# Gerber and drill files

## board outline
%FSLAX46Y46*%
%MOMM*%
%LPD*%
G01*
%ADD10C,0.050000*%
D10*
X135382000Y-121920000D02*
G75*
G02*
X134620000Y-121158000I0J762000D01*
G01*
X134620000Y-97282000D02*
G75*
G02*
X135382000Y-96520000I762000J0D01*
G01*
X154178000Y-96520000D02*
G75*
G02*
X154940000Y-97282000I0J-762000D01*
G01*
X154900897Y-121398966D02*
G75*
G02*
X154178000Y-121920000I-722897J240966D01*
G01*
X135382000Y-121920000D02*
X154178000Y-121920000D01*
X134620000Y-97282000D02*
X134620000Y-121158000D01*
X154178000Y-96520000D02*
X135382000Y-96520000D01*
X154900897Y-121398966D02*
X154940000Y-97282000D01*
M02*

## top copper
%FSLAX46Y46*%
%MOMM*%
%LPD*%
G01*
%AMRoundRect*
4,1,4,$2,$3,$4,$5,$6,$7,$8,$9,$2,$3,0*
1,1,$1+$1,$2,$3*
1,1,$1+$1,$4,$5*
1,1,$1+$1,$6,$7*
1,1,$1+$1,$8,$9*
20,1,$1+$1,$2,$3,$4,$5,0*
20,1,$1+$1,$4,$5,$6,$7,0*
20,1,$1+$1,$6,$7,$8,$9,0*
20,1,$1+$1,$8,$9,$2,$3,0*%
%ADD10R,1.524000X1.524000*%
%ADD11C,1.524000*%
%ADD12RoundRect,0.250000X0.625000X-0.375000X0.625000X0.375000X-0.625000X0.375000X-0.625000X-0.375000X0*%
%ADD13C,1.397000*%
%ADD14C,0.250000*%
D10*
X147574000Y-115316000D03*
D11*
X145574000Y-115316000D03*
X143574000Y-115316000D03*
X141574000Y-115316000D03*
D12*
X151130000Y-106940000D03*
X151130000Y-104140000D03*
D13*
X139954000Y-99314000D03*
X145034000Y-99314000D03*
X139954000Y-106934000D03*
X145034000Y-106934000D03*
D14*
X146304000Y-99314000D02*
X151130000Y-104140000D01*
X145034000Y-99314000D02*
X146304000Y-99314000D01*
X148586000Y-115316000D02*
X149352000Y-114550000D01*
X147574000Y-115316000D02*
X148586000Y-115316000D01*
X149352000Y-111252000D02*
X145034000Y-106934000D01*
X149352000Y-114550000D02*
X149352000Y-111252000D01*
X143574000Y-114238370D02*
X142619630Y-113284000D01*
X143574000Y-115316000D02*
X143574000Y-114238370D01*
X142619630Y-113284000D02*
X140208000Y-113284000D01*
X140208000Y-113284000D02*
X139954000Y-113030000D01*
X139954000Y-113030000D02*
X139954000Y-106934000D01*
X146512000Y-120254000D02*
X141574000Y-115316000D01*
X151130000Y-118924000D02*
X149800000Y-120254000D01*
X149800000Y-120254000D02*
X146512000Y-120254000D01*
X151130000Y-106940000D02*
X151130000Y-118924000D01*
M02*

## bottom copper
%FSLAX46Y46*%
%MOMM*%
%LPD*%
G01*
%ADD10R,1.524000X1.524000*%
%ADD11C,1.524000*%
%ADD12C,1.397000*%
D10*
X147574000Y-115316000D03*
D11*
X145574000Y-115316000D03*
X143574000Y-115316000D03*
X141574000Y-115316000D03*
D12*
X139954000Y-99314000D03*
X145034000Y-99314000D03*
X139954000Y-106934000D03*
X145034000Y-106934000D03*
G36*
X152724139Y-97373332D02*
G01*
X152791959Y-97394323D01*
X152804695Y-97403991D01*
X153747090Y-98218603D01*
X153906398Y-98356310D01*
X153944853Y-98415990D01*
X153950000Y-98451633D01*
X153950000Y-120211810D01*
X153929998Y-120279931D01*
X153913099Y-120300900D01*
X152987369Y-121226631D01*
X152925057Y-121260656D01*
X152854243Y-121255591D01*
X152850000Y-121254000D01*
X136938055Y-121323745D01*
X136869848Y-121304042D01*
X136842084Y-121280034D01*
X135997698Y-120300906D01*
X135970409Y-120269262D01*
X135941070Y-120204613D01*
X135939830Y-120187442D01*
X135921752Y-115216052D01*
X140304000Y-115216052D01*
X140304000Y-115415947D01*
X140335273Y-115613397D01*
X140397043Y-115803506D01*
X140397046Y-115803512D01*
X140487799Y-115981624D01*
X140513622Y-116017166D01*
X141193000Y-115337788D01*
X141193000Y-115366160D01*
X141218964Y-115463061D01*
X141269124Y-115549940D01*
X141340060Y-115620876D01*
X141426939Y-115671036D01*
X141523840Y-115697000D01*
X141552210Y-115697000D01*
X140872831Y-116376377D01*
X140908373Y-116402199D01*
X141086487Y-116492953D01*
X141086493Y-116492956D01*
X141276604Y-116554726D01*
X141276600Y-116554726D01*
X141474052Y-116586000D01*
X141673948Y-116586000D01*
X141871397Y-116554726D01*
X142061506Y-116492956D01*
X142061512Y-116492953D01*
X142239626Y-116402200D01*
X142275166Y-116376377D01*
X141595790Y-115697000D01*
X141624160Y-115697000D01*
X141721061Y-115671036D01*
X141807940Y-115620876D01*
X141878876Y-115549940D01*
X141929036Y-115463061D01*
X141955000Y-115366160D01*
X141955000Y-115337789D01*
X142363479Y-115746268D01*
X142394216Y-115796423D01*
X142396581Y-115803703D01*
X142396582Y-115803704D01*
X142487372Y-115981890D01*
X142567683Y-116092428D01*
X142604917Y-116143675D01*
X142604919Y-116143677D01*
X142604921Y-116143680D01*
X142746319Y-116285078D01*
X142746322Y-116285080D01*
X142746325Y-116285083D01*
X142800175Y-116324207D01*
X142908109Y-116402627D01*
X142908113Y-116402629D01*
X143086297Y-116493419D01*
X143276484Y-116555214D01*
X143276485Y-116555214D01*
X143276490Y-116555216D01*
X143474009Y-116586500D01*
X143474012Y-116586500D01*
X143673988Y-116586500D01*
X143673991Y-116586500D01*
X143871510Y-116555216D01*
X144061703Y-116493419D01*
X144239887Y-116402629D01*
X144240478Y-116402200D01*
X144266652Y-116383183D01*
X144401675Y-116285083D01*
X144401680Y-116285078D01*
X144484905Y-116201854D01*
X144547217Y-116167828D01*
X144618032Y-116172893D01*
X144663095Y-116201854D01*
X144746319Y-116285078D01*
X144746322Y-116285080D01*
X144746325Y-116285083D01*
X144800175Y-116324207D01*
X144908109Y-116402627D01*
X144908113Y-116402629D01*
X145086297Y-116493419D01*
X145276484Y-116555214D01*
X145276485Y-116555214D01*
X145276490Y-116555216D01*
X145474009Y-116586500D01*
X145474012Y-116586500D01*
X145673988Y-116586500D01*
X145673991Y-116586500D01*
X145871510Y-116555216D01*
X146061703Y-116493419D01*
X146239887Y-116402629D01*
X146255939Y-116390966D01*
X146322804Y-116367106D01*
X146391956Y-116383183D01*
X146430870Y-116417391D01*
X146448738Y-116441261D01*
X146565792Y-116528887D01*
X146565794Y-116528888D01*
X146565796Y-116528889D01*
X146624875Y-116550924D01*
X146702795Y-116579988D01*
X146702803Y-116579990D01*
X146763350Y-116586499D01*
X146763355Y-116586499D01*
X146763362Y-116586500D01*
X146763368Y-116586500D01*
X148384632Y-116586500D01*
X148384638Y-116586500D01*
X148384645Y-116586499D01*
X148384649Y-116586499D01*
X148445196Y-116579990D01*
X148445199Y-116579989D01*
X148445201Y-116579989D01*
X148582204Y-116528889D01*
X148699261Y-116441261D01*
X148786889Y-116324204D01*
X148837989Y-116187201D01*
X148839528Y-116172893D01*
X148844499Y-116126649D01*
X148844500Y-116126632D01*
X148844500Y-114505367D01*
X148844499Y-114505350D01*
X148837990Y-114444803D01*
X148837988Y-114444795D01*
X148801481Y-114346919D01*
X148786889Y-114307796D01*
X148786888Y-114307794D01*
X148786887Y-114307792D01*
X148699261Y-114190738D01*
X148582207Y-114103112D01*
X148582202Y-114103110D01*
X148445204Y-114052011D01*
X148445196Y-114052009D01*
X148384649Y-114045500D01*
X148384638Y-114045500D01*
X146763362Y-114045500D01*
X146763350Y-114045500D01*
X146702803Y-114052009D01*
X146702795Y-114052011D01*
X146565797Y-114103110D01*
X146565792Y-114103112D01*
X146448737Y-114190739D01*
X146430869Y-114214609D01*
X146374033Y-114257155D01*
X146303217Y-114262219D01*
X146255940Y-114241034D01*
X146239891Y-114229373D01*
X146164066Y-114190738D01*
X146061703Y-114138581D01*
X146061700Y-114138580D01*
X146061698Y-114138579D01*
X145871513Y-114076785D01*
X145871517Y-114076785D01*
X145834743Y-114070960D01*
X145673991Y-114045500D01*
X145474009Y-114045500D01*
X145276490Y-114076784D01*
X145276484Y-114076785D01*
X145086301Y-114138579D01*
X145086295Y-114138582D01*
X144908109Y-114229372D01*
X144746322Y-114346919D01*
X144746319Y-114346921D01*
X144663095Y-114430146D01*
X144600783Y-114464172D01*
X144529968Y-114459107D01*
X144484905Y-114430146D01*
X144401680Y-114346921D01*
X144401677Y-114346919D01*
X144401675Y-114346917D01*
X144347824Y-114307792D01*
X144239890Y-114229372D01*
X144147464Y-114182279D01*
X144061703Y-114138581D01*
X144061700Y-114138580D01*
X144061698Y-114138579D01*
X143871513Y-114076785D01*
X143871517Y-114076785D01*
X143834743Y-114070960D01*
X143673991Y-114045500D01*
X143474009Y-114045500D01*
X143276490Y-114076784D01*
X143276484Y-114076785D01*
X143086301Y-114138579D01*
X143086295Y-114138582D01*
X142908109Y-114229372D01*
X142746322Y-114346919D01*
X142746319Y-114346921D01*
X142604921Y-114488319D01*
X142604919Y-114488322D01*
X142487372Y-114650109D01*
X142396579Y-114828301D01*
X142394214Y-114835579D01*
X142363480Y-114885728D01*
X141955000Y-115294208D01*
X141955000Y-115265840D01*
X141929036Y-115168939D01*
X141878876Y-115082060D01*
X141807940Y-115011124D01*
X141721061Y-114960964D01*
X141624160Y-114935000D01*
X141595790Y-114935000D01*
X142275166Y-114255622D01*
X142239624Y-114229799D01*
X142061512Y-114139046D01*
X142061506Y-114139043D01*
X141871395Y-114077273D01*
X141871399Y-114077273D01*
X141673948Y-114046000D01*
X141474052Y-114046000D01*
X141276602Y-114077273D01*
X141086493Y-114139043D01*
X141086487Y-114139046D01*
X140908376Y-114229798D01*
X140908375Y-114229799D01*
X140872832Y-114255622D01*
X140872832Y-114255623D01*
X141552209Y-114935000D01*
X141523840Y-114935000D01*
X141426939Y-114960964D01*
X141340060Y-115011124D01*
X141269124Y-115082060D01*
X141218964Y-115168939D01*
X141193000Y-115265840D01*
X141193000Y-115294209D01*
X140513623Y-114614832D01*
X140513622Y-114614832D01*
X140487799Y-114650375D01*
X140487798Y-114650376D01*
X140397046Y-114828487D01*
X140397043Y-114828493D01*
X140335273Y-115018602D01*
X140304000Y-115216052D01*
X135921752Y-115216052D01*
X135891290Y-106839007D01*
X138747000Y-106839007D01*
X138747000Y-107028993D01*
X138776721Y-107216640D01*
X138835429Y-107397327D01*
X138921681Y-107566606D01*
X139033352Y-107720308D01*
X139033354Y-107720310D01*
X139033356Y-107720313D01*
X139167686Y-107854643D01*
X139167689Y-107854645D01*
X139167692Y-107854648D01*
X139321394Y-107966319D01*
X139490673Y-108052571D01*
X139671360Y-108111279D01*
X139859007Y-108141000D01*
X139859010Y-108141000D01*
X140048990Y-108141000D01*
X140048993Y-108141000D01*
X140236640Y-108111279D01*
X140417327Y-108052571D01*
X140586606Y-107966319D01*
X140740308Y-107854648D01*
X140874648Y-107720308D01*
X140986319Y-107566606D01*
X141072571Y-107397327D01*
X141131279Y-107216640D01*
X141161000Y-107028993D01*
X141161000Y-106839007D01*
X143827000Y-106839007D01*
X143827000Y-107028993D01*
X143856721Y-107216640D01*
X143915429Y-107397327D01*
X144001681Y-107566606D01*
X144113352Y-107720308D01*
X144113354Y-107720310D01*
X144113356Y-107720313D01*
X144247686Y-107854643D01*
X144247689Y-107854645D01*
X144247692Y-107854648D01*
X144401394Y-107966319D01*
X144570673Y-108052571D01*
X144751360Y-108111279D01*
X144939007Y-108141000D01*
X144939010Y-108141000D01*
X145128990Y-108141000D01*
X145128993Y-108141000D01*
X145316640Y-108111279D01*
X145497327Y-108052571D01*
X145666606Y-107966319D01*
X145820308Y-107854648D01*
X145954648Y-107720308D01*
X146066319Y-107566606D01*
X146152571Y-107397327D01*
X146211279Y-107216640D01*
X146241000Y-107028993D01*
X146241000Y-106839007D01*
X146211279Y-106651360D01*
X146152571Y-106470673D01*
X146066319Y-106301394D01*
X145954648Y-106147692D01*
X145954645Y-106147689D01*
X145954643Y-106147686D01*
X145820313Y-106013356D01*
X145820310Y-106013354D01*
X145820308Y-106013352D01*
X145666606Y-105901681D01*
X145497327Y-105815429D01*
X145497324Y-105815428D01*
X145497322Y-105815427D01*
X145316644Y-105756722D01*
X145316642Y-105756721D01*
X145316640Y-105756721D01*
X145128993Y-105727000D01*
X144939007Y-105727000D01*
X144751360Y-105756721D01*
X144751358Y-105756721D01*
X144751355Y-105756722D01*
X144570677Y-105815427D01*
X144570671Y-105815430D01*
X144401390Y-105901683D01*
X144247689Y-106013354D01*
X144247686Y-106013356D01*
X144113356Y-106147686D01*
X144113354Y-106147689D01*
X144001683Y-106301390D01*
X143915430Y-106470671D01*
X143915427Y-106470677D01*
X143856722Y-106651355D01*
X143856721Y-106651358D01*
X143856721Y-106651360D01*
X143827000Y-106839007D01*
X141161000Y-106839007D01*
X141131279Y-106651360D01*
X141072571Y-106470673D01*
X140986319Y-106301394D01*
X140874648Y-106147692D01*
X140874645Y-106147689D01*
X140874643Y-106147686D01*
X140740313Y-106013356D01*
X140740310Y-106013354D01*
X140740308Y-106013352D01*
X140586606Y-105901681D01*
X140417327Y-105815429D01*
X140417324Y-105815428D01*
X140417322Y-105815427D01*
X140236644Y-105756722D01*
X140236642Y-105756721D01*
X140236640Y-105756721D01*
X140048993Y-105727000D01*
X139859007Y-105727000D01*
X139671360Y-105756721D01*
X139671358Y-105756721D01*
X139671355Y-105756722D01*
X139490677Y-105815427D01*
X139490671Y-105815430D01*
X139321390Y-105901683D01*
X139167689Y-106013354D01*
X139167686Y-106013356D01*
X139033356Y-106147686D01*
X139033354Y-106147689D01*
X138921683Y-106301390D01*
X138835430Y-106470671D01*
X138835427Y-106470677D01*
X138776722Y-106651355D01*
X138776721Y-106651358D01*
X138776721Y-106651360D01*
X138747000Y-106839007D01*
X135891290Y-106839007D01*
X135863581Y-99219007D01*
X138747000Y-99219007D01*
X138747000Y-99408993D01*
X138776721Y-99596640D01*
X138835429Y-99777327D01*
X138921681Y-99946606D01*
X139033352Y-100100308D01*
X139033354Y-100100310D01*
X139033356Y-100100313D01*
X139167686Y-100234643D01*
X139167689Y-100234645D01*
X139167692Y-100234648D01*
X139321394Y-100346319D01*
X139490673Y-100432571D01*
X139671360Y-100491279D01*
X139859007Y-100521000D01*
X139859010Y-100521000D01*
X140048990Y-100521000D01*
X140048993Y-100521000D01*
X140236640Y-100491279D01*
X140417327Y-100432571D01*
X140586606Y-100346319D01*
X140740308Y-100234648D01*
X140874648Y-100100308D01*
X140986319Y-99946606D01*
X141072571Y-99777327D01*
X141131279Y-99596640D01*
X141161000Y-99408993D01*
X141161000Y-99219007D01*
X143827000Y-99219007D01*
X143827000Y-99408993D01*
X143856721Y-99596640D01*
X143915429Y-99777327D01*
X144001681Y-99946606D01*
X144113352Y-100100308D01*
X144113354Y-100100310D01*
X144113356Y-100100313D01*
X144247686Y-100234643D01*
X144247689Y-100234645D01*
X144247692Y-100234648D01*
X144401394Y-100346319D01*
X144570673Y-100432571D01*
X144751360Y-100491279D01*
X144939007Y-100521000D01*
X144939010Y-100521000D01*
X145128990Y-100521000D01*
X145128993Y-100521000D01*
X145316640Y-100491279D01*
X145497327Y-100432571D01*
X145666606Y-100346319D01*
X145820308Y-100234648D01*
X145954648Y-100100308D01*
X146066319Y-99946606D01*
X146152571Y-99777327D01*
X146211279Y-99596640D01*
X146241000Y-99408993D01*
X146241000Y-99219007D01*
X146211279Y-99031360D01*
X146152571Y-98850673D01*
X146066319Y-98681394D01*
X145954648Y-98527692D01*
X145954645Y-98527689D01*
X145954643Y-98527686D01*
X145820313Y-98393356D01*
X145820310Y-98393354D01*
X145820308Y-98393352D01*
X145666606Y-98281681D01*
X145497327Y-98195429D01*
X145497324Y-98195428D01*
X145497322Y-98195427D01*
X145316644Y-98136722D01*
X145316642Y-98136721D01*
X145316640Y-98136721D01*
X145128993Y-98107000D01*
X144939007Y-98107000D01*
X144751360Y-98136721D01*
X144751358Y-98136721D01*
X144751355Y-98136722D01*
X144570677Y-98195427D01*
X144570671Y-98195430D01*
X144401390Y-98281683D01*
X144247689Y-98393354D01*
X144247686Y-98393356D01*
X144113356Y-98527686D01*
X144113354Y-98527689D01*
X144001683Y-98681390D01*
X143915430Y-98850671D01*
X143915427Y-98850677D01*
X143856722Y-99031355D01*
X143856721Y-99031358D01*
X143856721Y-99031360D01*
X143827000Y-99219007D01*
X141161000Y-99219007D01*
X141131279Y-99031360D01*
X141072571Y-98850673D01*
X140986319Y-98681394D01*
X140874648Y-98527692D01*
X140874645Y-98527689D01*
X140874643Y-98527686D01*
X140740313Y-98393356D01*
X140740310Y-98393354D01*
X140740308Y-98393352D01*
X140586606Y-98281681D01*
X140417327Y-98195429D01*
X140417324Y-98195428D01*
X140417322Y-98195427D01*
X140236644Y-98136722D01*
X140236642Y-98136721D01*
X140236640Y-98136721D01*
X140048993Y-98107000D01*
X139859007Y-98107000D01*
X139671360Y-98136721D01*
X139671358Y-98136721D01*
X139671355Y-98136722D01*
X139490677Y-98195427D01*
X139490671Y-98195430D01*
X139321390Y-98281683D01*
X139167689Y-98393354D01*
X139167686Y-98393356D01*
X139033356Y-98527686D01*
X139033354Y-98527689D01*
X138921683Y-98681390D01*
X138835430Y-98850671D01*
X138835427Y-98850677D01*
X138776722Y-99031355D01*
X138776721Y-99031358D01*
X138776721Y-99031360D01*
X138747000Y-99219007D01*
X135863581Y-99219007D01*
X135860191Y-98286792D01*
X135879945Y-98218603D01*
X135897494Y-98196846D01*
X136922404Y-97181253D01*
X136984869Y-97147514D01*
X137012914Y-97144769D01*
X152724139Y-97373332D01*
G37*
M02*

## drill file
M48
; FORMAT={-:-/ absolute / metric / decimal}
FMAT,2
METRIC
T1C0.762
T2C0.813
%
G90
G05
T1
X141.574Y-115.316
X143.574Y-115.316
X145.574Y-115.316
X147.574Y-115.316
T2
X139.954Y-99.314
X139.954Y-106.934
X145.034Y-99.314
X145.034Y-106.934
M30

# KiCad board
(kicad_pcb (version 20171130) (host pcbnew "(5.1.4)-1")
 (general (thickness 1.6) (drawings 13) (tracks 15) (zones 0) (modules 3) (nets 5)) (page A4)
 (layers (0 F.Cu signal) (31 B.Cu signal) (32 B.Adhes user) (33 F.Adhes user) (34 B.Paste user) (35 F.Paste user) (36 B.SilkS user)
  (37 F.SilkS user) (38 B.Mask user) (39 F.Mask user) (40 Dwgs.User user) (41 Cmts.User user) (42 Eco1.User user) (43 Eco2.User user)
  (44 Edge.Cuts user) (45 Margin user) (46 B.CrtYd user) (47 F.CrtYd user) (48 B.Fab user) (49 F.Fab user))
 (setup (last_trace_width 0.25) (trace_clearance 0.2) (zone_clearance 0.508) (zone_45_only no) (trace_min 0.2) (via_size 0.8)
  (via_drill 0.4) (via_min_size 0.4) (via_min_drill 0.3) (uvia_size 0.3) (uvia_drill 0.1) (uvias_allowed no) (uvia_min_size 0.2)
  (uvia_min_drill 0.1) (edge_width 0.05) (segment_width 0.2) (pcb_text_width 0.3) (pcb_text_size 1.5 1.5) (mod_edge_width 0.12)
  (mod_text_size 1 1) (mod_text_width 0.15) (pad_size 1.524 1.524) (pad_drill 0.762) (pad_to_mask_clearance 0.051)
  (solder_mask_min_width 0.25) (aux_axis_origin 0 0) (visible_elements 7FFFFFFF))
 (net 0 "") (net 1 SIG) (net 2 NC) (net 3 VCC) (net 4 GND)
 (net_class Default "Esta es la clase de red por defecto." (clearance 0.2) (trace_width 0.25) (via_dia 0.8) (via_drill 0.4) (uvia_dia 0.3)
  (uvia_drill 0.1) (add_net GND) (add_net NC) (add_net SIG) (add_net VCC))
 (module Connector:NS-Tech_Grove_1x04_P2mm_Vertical (layer F.Cu) (at 147.574 115.316 270)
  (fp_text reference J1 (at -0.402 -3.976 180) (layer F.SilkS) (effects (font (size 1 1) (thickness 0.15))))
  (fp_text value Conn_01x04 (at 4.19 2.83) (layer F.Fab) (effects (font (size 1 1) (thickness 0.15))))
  (pad 1 thru_hole rect (at 0 0 270) (size 1.524 1.524) (drill 0.762) (layers *.Cu *.Mask) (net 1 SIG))
  (pad 2 thru_hole circle (at 0 2 270) (size 1.524 1.524) (drill 0.762) (layers *.Cu *.Mask) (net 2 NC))
  (pad 3 thru_hole circle (at 0 4 270) (size 1.524 1.524) (drill 0.762) (layers *.Cu *.Mask) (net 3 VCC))
  (pad 4 thru_hole circle (at 0 6 270) (size 1.524 1.524) (drill 0.762) (layers *.Cu *.Mask) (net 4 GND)))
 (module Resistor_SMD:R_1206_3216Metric (layer F.Cu) (at 151.13 105.54 90)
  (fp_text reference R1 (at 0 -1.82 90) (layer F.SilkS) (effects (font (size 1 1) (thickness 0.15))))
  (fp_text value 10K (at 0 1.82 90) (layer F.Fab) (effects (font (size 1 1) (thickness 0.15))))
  (pad 1 smd roundrect (at -1.4 0 90) (size 1.25 1.75) (layers F.Cu F.Paste F.Mask) (roundrect_rratio 0.2) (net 4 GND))
  (pad 2 smd roundrect (at 1.4 0 90) (size 1.25 1.75) (layers F.Cu F.Paste F.Mask) (roundrect_rratio 0.2) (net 1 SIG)))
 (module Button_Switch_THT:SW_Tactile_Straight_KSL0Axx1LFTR (layer F.Cu) (at 139.954 106.934 90)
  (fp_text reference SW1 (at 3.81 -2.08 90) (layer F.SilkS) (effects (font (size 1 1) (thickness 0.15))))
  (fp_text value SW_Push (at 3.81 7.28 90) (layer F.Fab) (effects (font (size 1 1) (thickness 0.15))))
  (pad 1 thru_hole circle (at 7.62 0 90) (size 1.397 1.397) (drill 0.8128) (layers *.Cu *.Mask) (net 3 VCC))
  (pad 2 thru_hole circle (at 7.62 5.08 90) (size 1.397 1.397) (drill 0.8128) (layers *.Cu *.Mask) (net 1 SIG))
  (pad 1 thru_hole circle (at 0 0 90) (size 1.397 1.397) (drill 0.8128) (layers *.Cu *.Mask) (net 3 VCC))
  (pad 2 thru_hole circle (at 0 5.08 90) (size 1.397 1.397) (drill 0.8128) (layers *.Cu *.Mask) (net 1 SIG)))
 (gr_arc (start 135.382 121.158) (end 134.62 121.158) (angle -90) (layer Edge.Cuts) (width 0.05))
 (gr_arc (start 135.382 97.282) (end 135.382 96.52) (angle -90) (layer Edge.Cuts) (width 0.05))
 (gr_arc (start 154.178 97.282) (end 154.94 97.282) (angle -90) (layer Edge.Cuts) (width 0.05))
 (gr_arc (start 154.178 121.158) (end 154.178 121.92) (angle -71.56505118) (layer Edge.Cuts) (width 0.05))
 (gr_line (start 135.382 121.92) (end 154.178 121.92) (layer Edge.Cuts) (width 0.05))
 (gr_line (start 134.62 97.282) (end 134.62 121.158) (layer Edge.Cuts) (width 0.05))
 (gr_line (start 154.178 96.52) (end 135.382 96.52) (layer Edge.Cuts) (width 0.05))
 (gr_line (start 154.900897 121.398966) (end 154.94 97.282) (layer Edge.Cuts) (width 0.05))
 (segment (start 146.304 99.314) (end 151.13 104.14) (width 0.25) (layer F.Cu) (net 1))
 (segment (start 145.034 99.314) (end 146.304 99.314) (width 0.25) (layer F.Cu) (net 1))
 (segment (start 148.586 115.316) (end 149.352 114.55) (width 0.25) (layer F.Cu) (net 1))
 (segment (start 147.574 115.316) (end 148.586 115.316) (width 0.25) (layer F.Cu) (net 1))
 (segment (start 149.352 111.252) (end 145.034 106.934) (width 0.25) (layer F.Cu) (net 1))
 (segment (start 149.352 114.55) (end 149.352 111.252) (width 0.25) (layer F.Cu) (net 1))
 (segment (start 143.574 114.23837) (end 142.61963 113.284) (width 0.25) (layer F.Cu) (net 3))
 (segment (start 143.574 115.316) (end 143.574 114.23837) (width 0.25) (layer F.Cu) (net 3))
 (segment (start 142.61963 113.284) (end 140.208 113.284) (width 0.25) (layer F.Cu) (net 3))
 (segment (start 140.208 113.284) (end 139.954 113.03) (width 0.25) (layer F.Cu) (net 3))
 (segment (start 139.954 113.03) (end 139.954 106.934) (width 0.25) (layer F.Cu) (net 3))
 (segment (start 146.512 120.254) (end 141.574 115.316) (width 0.25) (layer F.Cu) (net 4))
 (segment (start 151.13 118.924) (end 149.8 120.254) (width 0.25) (layer F.Cu) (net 4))
 (segment (start 149.8 120.254) (end 146.512 120.254) (width 0.25) (layer F.Cu) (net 4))
 (segment (start 151.13 106.94) (end 151.13 118.924) (width 0.25) (layer F.Cu) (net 4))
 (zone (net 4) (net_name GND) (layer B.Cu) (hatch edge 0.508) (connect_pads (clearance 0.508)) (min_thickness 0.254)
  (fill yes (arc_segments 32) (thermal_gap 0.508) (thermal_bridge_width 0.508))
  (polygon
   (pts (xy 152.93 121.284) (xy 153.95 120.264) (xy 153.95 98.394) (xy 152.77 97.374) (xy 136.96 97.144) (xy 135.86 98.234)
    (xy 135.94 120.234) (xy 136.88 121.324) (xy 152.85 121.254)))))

